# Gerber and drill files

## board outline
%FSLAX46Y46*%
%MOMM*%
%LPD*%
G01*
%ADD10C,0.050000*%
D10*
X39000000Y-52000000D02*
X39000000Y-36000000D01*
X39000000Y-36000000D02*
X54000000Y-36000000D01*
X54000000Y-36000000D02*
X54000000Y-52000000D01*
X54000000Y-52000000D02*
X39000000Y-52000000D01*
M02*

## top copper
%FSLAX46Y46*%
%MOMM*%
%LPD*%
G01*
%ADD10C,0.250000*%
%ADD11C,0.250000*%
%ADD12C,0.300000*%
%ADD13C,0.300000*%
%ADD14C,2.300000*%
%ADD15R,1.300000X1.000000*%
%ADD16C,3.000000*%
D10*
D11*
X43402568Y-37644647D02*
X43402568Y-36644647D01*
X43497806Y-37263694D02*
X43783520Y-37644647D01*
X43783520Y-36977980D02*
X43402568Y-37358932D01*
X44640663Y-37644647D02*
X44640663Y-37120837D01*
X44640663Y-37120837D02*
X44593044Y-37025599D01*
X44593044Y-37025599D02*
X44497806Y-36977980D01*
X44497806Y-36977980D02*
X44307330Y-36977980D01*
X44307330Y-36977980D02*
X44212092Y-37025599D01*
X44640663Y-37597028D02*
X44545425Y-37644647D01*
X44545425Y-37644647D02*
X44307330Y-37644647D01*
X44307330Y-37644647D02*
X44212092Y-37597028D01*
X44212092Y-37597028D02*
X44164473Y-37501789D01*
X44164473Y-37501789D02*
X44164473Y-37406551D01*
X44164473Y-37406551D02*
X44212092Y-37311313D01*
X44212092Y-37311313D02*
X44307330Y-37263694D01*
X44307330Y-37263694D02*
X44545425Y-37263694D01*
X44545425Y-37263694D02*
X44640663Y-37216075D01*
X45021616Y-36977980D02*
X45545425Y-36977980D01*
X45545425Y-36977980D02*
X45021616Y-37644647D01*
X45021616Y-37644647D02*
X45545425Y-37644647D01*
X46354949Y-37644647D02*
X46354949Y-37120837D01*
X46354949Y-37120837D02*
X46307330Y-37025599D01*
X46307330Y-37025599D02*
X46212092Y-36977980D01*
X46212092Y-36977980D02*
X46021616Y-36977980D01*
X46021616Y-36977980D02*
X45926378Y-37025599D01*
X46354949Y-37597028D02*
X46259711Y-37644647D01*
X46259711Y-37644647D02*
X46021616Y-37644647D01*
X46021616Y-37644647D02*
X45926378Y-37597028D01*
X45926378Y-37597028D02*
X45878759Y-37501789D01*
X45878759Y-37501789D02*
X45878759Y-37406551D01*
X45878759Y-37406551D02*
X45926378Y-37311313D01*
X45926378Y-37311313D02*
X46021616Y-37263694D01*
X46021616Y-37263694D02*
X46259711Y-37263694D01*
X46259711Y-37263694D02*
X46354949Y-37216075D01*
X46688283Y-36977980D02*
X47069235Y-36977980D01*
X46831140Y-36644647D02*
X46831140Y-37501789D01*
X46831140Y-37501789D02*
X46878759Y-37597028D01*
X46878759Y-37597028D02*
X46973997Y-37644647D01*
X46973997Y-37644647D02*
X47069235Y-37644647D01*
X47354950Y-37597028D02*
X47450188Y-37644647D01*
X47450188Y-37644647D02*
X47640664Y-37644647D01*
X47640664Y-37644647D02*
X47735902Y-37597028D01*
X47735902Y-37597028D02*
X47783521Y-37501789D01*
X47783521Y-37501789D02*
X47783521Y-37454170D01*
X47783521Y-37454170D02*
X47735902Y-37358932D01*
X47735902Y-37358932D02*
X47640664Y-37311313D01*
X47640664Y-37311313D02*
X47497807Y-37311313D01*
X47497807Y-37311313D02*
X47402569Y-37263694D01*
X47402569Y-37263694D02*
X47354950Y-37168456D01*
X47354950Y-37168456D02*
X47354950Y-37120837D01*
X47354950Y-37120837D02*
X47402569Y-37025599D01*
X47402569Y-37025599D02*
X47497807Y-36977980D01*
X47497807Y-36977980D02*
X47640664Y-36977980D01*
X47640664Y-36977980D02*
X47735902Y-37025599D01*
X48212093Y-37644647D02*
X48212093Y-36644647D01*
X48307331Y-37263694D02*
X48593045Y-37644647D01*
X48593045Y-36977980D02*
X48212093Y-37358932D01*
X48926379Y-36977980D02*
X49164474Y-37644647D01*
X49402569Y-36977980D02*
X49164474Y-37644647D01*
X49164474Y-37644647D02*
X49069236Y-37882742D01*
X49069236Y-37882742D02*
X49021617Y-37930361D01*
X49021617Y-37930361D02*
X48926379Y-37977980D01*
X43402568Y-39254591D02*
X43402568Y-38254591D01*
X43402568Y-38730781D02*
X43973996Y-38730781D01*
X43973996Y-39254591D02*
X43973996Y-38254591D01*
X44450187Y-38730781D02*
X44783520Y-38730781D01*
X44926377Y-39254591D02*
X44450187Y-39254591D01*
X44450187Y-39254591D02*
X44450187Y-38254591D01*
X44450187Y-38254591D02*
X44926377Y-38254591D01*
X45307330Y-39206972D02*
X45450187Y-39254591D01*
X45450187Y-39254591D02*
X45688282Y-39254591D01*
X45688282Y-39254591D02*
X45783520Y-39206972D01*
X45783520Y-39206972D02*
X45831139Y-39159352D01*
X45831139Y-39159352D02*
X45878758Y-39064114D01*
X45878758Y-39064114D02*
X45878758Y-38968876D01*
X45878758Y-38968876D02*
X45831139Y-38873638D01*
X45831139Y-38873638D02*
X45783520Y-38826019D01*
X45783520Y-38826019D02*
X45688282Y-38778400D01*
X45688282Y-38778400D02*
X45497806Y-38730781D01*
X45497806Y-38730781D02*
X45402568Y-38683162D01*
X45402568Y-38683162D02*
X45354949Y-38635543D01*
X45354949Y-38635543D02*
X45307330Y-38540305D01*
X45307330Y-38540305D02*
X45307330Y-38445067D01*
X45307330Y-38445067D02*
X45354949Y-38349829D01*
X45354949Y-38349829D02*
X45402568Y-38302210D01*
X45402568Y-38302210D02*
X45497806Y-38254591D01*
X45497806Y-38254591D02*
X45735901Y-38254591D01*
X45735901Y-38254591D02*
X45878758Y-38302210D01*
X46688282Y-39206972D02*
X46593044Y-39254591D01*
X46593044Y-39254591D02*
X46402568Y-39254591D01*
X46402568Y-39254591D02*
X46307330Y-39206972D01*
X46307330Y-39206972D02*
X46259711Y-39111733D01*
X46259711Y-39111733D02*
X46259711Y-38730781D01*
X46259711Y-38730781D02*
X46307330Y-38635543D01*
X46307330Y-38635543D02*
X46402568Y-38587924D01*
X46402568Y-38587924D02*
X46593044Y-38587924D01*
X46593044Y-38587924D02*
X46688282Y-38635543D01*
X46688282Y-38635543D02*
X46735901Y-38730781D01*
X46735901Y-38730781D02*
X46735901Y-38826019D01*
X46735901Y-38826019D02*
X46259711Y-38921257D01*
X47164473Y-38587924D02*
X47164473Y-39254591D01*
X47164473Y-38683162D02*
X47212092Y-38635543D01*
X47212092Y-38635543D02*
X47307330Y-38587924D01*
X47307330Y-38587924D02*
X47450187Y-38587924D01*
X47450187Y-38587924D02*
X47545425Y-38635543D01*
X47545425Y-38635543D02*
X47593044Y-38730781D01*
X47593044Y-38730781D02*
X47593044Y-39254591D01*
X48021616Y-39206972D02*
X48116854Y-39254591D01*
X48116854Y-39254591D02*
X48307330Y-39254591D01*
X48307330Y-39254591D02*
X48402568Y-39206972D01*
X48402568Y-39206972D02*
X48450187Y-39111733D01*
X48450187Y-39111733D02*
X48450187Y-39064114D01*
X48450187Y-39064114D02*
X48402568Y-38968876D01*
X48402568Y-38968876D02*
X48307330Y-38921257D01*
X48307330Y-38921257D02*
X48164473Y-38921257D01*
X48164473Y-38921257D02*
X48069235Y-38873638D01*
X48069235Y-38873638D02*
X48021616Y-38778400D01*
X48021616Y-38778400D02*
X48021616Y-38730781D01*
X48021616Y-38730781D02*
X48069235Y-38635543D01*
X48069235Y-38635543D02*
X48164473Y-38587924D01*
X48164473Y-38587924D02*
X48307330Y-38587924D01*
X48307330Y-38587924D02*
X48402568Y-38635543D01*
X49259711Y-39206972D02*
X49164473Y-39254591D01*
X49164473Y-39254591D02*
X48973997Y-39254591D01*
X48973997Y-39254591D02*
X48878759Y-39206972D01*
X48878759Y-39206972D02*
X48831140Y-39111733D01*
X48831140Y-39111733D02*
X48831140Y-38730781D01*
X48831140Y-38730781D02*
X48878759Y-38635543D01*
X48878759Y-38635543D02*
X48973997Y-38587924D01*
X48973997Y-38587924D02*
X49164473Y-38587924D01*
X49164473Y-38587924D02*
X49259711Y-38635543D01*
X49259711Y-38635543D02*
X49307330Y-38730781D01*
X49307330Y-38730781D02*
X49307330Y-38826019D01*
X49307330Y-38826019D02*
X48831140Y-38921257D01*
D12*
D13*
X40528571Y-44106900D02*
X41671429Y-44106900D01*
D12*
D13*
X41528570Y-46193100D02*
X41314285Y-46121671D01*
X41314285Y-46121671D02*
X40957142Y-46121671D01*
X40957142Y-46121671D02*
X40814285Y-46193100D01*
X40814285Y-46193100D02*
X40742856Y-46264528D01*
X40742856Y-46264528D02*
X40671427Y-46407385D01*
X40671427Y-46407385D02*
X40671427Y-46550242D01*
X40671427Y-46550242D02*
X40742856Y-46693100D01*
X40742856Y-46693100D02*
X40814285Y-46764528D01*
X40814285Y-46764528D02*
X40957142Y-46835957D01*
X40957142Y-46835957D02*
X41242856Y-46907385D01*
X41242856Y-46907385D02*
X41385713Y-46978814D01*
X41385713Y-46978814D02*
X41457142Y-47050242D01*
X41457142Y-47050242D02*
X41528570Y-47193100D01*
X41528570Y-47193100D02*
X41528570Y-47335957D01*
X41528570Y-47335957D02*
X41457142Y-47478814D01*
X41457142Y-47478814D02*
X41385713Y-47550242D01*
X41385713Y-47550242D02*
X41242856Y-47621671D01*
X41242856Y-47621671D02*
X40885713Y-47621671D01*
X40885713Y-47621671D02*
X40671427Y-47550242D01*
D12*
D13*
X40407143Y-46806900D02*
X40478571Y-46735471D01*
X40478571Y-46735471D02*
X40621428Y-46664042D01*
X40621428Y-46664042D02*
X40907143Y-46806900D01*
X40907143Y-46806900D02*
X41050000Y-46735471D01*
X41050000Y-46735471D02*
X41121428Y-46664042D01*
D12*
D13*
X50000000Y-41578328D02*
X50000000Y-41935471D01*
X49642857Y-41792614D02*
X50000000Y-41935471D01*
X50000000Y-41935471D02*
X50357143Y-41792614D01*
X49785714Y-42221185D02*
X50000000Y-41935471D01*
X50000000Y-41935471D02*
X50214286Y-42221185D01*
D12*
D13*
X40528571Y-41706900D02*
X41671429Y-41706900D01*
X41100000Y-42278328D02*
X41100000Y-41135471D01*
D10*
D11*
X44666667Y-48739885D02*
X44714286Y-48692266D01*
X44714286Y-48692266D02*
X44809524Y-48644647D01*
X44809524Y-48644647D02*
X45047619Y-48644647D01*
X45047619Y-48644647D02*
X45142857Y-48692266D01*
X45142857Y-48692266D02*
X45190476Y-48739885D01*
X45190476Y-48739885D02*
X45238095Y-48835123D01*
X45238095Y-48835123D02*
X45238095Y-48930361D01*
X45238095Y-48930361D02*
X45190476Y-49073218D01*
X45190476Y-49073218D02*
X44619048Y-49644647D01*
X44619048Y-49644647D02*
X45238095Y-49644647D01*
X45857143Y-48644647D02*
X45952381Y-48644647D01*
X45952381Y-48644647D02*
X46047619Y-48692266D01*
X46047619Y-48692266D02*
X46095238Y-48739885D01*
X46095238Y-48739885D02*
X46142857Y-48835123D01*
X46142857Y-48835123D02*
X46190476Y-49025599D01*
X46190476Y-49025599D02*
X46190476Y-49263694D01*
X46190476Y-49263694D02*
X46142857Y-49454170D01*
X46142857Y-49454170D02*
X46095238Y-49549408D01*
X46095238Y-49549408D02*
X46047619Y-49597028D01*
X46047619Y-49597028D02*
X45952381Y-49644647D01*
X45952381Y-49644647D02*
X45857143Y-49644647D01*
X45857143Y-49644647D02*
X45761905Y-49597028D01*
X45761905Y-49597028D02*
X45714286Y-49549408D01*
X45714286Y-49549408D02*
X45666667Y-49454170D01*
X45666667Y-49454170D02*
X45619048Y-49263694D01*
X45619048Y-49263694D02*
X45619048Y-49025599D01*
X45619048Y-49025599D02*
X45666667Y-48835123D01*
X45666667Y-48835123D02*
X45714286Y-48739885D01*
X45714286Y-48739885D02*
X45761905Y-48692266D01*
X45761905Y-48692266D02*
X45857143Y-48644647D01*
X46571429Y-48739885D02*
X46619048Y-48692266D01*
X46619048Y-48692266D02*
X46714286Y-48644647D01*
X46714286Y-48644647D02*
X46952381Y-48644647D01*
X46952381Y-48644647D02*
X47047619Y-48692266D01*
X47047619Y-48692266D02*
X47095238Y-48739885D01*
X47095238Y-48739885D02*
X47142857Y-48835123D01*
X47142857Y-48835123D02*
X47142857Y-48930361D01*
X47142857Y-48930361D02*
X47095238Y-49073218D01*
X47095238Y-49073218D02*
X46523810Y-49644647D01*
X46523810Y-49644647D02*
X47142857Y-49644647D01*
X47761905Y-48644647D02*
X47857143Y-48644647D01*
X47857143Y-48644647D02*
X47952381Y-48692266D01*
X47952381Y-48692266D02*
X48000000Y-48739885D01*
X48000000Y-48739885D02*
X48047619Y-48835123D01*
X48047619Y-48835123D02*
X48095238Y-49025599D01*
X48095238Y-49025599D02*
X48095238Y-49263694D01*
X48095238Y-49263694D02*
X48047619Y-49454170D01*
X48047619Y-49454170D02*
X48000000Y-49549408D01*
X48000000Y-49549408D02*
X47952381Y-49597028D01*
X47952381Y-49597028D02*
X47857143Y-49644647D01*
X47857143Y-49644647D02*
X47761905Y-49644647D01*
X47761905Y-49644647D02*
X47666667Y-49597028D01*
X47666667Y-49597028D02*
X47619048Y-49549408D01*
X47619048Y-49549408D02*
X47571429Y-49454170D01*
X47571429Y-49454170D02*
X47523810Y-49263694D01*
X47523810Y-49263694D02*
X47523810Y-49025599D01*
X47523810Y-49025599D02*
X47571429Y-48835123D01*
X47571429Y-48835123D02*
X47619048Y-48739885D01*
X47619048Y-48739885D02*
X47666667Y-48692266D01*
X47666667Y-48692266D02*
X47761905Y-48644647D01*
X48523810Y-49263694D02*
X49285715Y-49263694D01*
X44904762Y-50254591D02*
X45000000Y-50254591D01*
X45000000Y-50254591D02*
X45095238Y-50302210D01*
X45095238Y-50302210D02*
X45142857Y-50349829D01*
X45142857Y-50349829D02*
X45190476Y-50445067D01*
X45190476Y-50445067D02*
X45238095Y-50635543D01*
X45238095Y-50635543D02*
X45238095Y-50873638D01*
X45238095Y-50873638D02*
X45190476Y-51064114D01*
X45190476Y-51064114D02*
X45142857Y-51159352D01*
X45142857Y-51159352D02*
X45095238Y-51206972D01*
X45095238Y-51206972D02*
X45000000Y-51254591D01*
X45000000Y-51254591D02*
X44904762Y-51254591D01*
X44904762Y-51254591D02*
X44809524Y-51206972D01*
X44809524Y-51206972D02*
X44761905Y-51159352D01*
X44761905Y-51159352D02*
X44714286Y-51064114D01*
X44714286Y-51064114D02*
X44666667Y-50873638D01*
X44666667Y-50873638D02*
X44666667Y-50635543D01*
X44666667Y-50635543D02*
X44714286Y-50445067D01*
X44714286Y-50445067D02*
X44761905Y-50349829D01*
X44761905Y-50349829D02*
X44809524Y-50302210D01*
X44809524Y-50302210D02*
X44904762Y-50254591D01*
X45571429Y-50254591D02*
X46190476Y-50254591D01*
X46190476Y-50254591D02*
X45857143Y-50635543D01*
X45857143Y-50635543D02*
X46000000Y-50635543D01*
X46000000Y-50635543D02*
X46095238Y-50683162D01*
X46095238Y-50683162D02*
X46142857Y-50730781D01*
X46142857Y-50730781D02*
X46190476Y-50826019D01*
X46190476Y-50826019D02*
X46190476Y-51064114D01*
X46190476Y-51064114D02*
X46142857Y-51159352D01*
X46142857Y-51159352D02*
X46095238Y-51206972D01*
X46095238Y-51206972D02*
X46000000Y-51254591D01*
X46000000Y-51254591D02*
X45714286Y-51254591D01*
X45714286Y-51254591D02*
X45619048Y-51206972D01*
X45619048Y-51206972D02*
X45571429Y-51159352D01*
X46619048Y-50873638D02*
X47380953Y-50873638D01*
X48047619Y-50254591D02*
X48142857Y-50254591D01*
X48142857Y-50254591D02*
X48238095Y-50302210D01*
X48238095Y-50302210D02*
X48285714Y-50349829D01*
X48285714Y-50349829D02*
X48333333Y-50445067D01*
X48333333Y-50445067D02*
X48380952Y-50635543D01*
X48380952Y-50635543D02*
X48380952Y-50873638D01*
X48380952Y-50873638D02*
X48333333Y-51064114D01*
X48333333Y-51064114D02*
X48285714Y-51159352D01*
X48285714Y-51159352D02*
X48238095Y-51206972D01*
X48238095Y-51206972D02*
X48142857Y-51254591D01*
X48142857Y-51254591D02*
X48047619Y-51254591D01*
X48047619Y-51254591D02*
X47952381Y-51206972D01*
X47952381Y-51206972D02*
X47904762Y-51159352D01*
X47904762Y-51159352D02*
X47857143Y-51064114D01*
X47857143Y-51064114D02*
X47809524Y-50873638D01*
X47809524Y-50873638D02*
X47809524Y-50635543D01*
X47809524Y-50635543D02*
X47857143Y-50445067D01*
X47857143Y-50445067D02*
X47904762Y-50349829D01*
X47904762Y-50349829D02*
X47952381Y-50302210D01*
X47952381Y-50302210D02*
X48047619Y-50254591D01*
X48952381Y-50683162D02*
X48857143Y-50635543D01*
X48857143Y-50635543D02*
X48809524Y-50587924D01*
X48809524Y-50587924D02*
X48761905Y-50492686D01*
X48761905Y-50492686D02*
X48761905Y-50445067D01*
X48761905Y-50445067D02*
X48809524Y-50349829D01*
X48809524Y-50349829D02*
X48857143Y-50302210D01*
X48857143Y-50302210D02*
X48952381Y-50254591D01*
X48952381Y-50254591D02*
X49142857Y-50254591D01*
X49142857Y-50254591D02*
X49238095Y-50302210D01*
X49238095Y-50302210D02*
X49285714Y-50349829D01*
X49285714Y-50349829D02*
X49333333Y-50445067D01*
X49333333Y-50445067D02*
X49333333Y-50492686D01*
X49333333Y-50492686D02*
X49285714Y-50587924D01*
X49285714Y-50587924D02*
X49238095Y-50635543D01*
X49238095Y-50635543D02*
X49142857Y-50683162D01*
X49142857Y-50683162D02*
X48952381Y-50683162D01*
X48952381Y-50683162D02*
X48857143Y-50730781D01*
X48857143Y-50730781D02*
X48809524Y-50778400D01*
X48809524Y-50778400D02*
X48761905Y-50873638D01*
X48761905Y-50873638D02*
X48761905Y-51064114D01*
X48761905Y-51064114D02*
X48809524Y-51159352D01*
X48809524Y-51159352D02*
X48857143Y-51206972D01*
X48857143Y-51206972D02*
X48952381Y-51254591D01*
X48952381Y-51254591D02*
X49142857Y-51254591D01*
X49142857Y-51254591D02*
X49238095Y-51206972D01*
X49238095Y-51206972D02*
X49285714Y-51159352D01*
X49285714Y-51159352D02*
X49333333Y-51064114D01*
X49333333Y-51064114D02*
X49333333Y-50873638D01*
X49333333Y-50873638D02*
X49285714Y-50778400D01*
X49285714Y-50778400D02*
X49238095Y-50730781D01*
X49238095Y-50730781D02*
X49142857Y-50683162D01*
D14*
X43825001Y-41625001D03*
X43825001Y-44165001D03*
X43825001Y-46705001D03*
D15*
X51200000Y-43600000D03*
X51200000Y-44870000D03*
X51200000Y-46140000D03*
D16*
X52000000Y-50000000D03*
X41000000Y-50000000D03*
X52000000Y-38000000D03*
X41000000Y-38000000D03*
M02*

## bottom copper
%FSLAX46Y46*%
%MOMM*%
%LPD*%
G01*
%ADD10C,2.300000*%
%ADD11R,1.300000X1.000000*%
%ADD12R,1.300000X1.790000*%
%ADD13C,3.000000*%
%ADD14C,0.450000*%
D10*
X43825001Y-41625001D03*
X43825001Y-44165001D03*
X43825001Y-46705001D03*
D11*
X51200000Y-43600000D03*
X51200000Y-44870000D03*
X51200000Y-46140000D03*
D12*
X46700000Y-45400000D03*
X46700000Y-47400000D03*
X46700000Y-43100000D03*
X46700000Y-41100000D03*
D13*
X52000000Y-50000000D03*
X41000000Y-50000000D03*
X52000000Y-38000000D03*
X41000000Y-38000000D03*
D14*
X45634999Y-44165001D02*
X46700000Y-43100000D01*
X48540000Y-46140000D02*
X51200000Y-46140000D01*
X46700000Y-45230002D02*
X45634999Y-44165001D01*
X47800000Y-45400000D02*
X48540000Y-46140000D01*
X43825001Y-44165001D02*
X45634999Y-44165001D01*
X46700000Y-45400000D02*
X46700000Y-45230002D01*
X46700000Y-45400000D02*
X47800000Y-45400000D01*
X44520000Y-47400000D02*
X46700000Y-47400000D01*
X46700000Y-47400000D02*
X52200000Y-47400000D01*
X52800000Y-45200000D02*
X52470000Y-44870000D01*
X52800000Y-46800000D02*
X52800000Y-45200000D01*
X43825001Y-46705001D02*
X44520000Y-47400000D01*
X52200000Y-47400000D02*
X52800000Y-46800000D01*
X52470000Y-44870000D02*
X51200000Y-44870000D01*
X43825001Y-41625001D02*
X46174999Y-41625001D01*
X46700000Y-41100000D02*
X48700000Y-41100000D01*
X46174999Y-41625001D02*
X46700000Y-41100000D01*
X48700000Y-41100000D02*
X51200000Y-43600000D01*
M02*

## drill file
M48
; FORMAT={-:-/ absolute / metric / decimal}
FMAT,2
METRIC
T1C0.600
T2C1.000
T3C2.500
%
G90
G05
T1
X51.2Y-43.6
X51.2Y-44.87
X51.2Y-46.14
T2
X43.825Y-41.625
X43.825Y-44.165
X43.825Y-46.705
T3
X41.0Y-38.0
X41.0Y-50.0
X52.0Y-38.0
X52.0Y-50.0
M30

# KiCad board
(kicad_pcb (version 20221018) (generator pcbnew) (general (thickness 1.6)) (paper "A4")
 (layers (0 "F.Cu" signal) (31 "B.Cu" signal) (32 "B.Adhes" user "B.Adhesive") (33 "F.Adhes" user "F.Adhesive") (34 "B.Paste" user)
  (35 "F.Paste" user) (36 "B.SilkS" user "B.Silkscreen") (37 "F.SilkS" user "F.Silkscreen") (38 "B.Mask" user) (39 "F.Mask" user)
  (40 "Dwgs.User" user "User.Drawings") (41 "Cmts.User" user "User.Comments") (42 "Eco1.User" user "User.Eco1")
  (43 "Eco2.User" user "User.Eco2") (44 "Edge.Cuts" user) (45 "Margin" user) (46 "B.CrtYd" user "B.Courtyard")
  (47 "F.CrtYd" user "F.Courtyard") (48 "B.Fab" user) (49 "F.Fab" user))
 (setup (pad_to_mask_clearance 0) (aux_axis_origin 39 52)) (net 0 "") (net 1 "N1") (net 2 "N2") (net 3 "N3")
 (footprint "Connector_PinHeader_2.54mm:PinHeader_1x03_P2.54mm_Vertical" (layer "F.Cu") (at 43.825001 41.625001)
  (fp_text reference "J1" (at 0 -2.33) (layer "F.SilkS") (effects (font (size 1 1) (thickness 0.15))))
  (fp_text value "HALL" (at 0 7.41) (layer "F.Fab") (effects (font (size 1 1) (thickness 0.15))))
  (pad "1" thru_hole circle (at 0 0) (size 2.3 2.3) (drill 1) (layers "*.Cu" "*.Mask") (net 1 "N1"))
  (pad "2" thru_hole circle (at 0 2.54) (size 2.3 2.3) (drill 1) (layers "*.Cu" "*.Mask") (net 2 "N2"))
  (pad "3" thru_hole circle (at 0 5.08) (size 2.3 2.3) (drill 1) (layers "*.Cu" "*.Mask") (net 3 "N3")))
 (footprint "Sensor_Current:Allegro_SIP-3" (layer "F.Cu") (at 51.2 43.6 -90)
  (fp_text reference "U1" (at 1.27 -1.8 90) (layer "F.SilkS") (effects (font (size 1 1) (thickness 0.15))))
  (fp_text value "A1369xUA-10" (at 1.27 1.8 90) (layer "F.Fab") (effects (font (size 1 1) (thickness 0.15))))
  (pad "1" thru_hole rect (at 0 0 270) (size 1 1.3) (drill 0.6) (layers "*.Cu" "*.Mask") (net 1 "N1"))
  (pad "2" thru_hole rect (at 1.27 0 270) (size 1 1.3) (drill 0.6) (layers "*.Cu" "*.Mask") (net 3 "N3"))
  (pad "3" thru_hole rect (at 2.54 0 270) (size 1 1.3) (drill 0.6) (layers "*.Cu" "*.Mask") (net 2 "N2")))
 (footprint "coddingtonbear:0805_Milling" (layer "B.Cu") (at 46.7 46.4 -90)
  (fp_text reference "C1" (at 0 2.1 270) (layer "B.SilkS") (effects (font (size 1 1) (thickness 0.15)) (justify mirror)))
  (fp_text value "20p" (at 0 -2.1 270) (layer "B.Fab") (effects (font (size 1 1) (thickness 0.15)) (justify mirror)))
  (pad "1" smd rect (at -1 0 270) (size 1.79 1.3) (layers "B.Cu" "B.Paste" "B.Mask") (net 2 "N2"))
  (pad "2" smd rect (at 1 0 270) (size 1.79 1.3) (layers "B.Cu" "B.Paste" "B.Mask") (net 3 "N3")))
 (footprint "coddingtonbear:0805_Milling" (layer "B.Cu") (at 46.7 42.1 90)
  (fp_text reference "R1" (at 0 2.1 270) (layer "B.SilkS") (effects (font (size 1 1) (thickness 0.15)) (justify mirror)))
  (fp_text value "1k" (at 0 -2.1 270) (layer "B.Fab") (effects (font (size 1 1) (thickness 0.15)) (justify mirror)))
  (pad "1" smd rect (at -1 0 90) (size 1.79 1.3) (layers "B.Cu" "B.Paste" "B.Mask") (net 2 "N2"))
  (pad "2" smd rect (at 1 0 90) (size 1.79 1.3) (layers "B.Cu" "B.Paste" "B.Mask") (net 1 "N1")))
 (gr_line (start 39 52) (end 39 36) (stroke (width 0.05) (type solid)) (layer "Edge.Cuts"))
 (gr_line (start 39 36) (end 54 36) (stroke (width 0.05) (type solid)) (layer "Edge.Cuts"))
 (gr_line (start 54 36) (end 54 52) (stroke (width 0.05) (type solid)) (layer "Edge.Cuts"))
 (gr_line (start 54 52) (end 39 52) (stroke (width 0.05) (type solid)) (layer "Edge.Cuts"))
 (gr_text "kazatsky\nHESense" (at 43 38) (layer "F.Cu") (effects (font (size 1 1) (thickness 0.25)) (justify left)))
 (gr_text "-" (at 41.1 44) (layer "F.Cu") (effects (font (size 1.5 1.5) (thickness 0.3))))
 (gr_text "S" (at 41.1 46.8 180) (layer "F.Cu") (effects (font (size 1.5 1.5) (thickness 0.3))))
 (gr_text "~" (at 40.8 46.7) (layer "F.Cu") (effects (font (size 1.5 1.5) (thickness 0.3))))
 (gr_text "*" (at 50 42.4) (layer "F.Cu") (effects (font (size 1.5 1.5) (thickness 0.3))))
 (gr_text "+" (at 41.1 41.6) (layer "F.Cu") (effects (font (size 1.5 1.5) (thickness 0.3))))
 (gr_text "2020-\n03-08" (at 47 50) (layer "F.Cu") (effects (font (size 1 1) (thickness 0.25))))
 (via (at 52 50) (size 3) (drill 2.5) (layers "F.Cu" "B.Cu") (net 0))
 (via (at 41 50) (size 3) (drill 2.5) (layers "F.Cu" "B.Cu") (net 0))
 (via (at 52 38) (size 3) (drill 2.5) (layers "F.Cu" "B.Cu") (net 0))
 (via (at 41 38) (size 3) (drill 2.5) (layers "F.Cu" "B.Cu") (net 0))
 (segment (start 45.634999 44.165001) (end 46.7 43.1) (width 0.45) (layer "B.Cu") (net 2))
 (segment (start 48.54 46.14) (end 51.2 46.14) (width 0.45) (layer "B.Cu") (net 2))
 (segment (start 46.7 45.230002) (end 45.634999 44.165001) (width 0.45) (layer "B.Cu") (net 2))
 (segment (start 47.8 45.4) (end 48.54 46.14) (width 0.45) (layer "B.Cu") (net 2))
 (segment (start 43.825001 44.165001) (end 45.634999 44.165001) (width 0.45) (layer "B.Cu") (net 2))
 (segment (start 46.7 45.4) (end 46.7 45.230002) (width 0.45) (layer "B.Cu") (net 2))
 (segment (start 46.7 45.4) (end 47.8 45.4) (width 0.45) (layer "B.Cu") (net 2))
 (segment (start 44.52 47.4) (end 46.7 47.4) (width 0.45) (layer "B.Cu") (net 3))
 (segment (start 46.7 47.4) (end 52.2 47.4) (width 0.45) (layer "B.Cu") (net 3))
 (segment (start 52.8 45.2) (end 52.47 44.87) (width 0.45) (layer "B.Cu") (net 3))
 (segment (start 52.8 46.8) (end 52.8 45.2) (width 0.45) (layer "B.Cu") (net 3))
 (segment (start 43.825001 46.705001) (end 44.52 47.4) (width 0.45) (layer "B.Cu") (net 3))
 (segment (start 52.2 47.4) (end 52.8 46.8) (width 0.45) (layer "B.Cu") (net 3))
 (segment (start 52.47 44.87) (end 51.2 44.87) (width 0.45) (layer "B.Cu") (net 3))
 (segment (start 43.825001 41.625001) (end 46.174999 41.625001) (width 0.45) (layer "B.Cu") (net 1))
 (segment (start 46.7 41.1) (end 48.7 41.1) (width 0.45) (layer "B.Cu") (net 1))
 (segment (start 46.174999 41.625001) (end 46.7 41.1) (width 0.45) (layer "B.Cu") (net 1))
 (segment (start 48.7 41.1) (end 51.2 43.6) (width 0.45) (layer "B.Cu") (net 1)))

